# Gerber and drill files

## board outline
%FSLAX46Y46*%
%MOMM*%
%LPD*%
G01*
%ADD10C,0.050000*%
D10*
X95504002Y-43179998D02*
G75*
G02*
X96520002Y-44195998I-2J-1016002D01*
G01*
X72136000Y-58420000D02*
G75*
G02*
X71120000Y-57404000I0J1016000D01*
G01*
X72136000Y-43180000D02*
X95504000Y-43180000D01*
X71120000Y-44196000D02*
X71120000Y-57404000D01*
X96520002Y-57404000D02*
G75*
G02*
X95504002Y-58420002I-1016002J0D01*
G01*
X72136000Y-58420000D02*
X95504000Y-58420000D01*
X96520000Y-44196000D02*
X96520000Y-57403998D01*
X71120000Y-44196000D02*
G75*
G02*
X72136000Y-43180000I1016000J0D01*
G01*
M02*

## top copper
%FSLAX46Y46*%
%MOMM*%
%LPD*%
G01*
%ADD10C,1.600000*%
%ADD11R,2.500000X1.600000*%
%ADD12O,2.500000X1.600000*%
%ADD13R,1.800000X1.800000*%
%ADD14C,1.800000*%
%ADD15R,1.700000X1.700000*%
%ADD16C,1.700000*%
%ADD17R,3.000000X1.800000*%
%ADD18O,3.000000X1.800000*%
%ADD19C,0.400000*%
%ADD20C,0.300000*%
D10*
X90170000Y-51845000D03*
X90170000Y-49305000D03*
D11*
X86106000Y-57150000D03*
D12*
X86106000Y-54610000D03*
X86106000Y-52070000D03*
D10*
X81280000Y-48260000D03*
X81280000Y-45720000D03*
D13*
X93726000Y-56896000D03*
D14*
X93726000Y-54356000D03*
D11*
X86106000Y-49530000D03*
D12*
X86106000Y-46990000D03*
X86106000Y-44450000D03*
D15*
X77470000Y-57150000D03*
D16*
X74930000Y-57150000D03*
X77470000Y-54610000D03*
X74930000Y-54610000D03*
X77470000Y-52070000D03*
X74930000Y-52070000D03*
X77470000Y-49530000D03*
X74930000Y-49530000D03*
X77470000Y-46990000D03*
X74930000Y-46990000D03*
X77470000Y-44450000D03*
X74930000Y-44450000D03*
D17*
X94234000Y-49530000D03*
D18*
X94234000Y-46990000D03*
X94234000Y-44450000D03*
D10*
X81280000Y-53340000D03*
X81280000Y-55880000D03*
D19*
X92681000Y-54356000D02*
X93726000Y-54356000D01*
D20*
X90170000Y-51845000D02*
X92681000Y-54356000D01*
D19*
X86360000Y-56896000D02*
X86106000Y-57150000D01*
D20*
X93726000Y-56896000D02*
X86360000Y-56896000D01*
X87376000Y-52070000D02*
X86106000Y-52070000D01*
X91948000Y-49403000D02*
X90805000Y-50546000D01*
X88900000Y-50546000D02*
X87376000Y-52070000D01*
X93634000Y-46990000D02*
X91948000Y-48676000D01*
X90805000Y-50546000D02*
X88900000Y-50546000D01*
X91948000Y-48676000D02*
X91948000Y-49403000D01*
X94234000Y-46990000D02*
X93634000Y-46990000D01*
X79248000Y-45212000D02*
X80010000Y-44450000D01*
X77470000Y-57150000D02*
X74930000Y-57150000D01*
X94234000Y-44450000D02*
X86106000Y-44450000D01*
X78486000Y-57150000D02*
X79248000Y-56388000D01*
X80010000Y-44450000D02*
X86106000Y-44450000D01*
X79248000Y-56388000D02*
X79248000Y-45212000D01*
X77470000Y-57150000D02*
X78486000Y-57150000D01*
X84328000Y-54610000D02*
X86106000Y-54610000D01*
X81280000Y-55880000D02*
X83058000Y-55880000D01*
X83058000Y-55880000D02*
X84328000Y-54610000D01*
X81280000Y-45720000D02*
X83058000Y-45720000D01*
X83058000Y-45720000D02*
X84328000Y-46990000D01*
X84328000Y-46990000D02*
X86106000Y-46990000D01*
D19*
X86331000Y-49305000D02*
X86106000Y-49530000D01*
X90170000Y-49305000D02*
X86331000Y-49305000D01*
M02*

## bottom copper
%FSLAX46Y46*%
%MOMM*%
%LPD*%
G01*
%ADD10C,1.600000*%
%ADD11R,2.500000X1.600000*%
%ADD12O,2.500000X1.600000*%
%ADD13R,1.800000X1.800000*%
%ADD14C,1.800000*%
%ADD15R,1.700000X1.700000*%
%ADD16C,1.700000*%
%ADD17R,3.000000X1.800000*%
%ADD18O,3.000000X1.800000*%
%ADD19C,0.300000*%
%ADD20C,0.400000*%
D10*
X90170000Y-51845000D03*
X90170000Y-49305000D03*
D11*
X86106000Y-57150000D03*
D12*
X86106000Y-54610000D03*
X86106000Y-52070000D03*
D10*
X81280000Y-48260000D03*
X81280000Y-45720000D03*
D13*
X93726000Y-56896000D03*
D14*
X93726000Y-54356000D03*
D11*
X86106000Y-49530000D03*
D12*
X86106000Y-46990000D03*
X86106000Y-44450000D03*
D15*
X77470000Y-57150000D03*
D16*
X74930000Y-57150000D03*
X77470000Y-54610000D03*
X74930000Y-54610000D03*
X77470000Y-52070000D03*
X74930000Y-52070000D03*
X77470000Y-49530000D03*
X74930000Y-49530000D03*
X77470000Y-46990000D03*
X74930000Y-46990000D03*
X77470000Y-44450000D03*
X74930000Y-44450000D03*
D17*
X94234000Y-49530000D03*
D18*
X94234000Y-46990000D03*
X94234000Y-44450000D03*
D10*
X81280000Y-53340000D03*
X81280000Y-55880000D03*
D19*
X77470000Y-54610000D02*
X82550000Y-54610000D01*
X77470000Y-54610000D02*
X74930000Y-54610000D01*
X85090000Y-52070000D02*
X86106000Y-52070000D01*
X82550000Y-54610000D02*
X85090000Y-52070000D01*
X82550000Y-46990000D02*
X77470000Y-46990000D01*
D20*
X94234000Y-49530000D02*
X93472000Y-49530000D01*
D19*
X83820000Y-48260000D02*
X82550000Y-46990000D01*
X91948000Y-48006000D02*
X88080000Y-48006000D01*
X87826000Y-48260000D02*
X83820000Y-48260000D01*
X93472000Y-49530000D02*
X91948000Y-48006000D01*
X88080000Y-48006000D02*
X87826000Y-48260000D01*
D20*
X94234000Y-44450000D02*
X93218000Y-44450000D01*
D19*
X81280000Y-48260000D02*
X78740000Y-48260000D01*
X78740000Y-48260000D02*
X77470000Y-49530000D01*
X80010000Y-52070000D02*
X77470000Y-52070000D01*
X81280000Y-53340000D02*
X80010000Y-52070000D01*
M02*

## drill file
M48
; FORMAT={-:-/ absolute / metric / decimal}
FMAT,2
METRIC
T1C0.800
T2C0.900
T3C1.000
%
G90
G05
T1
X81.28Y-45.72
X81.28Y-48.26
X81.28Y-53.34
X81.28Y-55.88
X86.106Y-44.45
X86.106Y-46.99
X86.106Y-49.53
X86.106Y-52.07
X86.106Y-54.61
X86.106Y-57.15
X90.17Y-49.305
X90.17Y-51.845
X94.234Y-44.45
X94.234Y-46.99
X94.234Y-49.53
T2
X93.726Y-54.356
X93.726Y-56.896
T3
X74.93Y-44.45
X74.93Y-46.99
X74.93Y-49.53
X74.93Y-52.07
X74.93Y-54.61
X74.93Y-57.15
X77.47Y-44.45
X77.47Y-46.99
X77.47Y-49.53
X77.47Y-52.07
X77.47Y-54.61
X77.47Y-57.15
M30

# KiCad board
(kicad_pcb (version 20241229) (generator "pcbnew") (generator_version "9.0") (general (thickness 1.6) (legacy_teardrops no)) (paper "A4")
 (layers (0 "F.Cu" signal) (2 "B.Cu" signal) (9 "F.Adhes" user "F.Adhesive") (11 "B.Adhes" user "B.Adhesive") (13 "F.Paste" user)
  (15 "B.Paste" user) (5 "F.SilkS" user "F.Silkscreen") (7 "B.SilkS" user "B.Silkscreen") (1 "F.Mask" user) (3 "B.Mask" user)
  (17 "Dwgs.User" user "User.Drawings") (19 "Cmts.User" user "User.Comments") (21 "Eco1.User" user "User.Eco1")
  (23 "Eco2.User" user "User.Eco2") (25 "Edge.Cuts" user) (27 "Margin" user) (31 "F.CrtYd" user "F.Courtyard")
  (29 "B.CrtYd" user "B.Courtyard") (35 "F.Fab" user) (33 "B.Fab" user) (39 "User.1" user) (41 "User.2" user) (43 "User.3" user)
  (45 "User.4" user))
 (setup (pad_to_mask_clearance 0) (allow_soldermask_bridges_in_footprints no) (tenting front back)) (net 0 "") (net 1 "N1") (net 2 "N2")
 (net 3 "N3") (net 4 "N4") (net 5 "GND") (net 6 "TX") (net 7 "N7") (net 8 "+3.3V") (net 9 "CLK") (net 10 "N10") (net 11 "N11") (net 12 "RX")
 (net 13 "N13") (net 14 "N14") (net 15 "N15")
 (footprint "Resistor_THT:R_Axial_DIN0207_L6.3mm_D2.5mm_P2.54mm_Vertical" (layer "F.Cu") (at 90.17 51.845 90)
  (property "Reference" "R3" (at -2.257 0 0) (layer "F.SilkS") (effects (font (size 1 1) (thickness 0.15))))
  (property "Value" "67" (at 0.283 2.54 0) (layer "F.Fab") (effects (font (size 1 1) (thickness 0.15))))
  (pad "1" thru_hole circle (at 0 0 90) (size 1.6 1.6) (drill 0.8) (layers "*.Cu" "*.Mask") (remove_unused_layers no) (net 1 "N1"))
  (pad "2" thru_hole circle (at 2.54 0 90) (size 1.6 1.6) (drill 0.8) (layers "*.Cu" "*.Mask") (remove_unused_layers no) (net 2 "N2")))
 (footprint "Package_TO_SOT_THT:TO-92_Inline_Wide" (layer "F.Cu") (at 86.106 57.15 90)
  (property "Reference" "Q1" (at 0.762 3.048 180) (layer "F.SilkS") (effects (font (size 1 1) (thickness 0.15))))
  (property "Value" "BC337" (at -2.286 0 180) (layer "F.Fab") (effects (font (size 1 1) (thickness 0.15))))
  (pad "1" thru_hole rect (at 0 0 90) (size 1.6 2.5) (drill 0.8) (layers "*.Cu" "*.Mask") (remove_unused_layers no) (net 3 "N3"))
  (pad "2" thru_hole oval (at 2.54 0 90) (size 1.6 2.5) (drill 0.8) (layers "*.Cu" "*.Mask") (remove_unused_layers no) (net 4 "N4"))
  (pad "3" thru_hole oval (at 5.08 0 90) (size 1.6 2.5) (drill 0.8) (layers "*.Cu" "*.Mask") (remove_unused_layers no) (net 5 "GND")))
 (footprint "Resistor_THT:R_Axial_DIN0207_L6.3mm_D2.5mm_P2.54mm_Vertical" (layer "F.Cu") (at 81.28 48.26 90)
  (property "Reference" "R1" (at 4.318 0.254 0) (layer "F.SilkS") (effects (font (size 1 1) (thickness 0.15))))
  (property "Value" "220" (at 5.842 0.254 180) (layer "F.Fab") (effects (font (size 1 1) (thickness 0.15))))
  (pad "1" thru_hole circle (at 0 0 90) (size 1.6 1.6) (drill 0.8) (layers "*.Cu" "*.Mask") (remove_unused_layers no) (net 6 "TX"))
  (pad "2" thru_hole circle (at 2.54 0 90) (size 1.6 1.6) (drill 0.8) (layers "*.Cu" "*.Mask") (remove_unused_layers no) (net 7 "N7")))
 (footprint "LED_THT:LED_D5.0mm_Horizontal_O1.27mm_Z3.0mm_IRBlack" (layer "F.Cu") (at 93.726 56.896 90)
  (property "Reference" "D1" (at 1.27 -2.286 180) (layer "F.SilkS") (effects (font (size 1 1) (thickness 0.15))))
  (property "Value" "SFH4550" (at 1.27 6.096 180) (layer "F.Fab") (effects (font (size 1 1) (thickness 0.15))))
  (pad "1" thru_hole rect (at 0 0 90) (size 1.8 1.8) (drill 0.9) (layers "*.Cu" "*.Mask") (remove_unused_layers no) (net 3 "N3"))
  (pad "2" thru_hole circle (at 2.54 0 90) (size 1.8 1.8) (drill 0.9) (layers "*.Cu" "*.Mask") (remove_unused_layers no) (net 1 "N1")))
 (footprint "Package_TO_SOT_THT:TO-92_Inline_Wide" (layer "F.Cu") (at 86.106 49.53 90)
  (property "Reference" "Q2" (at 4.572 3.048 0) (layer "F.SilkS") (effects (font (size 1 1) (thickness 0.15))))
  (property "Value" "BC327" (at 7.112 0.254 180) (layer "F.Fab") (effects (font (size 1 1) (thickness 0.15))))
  (pad "1" thru_hole rect (at 0 0 90) (size 1.6 2.5) (drill 0.8) (layers "*.Cu" "*.Mask") (remove_unused_layers no) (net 2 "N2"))
  (pad "2" thru_hole oval (at 2.54 0 90) (size 1.6 2.5) (drill 0.8) (layers "*.Cu" "*.Mask") (remove_unused_layers no) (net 7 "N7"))
  (pad "3" thru_hole oval (at 5.08 0 90) (size 1.6 2.5) (drill 0.8) (layers "*.Cu" "*.Mask") (remove_unused_layers no) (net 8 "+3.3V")))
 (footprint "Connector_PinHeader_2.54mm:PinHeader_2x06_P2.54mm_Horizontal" (layer "F.Cu") (at 77.47 57.15 180)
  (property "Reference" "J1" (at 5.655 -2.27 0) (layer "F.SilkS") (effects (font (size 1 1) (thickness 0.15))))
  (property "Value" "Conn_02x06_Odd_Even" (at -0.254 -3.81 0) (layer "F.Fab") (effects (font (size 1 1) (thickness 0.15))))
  (pad "1" thru_hole rect (at 0 0 180) (size 1.7 1.7) (drill 1) (layers "*.Cu" "*.Mask") (remove_unused_layers no) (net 8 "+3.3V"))
  (pad "2" thru_hole circle (at 2.54 0 180) (size 1.7 1.7) (drill 1) (layers "*.Cu" "*.Mask") (remove_unused_layers no) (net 8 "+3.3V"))
  (pad "3" thru_hole circle (at 0 2.54 180) (size 1.7 1.7) (drill 1) (layers "*.Cu" "*.Mask") (remove_unused_layers no) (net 5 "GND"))
  (pad "4" thru_hole circle (at 2.54 2.54 180) (size 1.7 1.7) (drill 1) (layers "*.Cu" "*.Mask") (remove_unused_layers no) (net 5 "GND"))
  (pad "5" thru_hole circle (at 0 5.08 180) (size 1.7 1.7) (drill 1) (layers "*.Cu" "*.Mask") (remove_unused_layers no) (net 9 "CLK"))
  (pad "6" thru_hole circle (at 2.54 5.08 180) (size 1.7 1.7) (drill 1) (layers "*.Cu" "*.Mask") (remove_unused_layers no) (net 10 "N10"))
  (pad "7" thru_hole circle (at 0 7.62 180) (size 1.7 1.7) (drill 1) (layers "*.Cu" "*.Mask") (remove_unused_layers no) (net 6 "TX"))
  (pad "8" thru_hole circle (at 2.54 7.62 180) (size 1.7 1.7) (drill 1) (layers "*.Cu" "*.Mask") (remove_unused_layers no) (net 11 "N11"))
  (pad "9" thru_hole circle (at 0 10.16 180) (size 1.7 1.7) (drill 1) (layers "*.Cu" "*.Mask") (remove_unused_layers no) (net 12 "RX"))
  (pad "10" thru_hole circle (at 2.54 10.16 180) (size 1.7 1.7) (drill 1) (layers "*.Cu" "*.Mask") (remove_unused_layers no) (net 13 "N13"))
  (pad "11" thru_hole circle (at 0 12.7 180) (size 1.7 1.7) (drill 1) (layers "*.Cu" "*.Mask") (remove_unused_layers no) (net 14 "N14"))
  (pad "12" thru_hole circle (at 2.54 12.7 180) (size 1.7 1.7) (drill 1) (layers "*.Cu" "*.Mask") (remove_unused_layers no) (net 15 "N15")))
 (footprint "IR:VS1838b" (layer "F.Cu") (at 94.234 46.99 180)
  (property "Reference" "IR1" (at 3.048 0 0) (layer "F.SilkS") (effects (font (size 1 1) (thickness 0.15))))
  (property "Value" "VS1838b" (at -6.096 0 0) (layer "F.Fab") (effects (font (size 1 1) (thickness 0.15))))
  (pad "1" thru_hole rect (at 0 -2.54 180) (size 3 1.8) (drill 0.8) (layers "*.Cu" "*.Mask") (remove_unused_layers no) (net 12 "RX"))
  (pad "2" thru_hole oval (at 0 0 180) (size 3 1.8) (drill 0.8) (layers "*.Cu" "*.Mask") (remove_unused_layers no) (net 5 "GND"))
  (pad "3" thru_hole oval (at 0 2.54 180) (size 3 1.8) (drill 0.8) (layers "*.Cu" "*.Mask") (remove_unused_layers no) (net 8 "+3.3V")))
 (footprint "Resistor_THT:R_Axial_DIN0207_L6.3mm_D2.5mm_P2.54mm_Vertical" (layer "F.Cu") (at 81.28 53.34 -90)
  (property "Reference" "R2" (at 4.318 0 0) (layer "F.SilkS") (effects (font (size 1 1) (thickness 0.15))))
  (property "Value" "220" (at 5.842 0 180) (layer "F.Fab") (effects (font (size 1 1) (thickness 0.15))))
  (pad "1" thru_hole circle (at 0 0 270) (size 1.6 1.6) (drill 0.8) (layers "*.Cu" "*.Mask") (remove_unused_layers no) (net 9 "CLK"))
  (pad "2" thru_hole circle (at 2.54 0 270) (size 1.6 1.6) (drill 0.8) (layers "*.Cu" "*.Mask") (remove_unused_layers no) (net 4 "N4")))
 (gr_arc (start 95.504002 43.179998) (mid 96.222422 43.477578) (end 96.520002 44.195998) (stroke (width 0.05) (type default))
  (layer "Edge.Cuts"))
 (gr_arc (start 72.136 58.42) (mid 71.41758 58.12242) (end 71.12 57.404) (stroke (width 0.05) (type default)) (layer "Edge.Cuts"))
 (gr_line (start 72.136 43.18) (end 95.504 43.18) (stroke (width 0.05) (type default)) (layer "Edge.Cuts"))
 (gr_line (start 71.12 44.196) (end 71.12 57.404) (stroke (width 0.05) (type default)) (layer "Edge.Cuts"))
 (gr_arc (start 96.520002 57.404) (mid 96.222422 58.12242) (end 95.504002 58.42) (stroke (width 0.05) (type default)) (layer "Edge.Cuts"))
 (gr_line (start 72.136 58.42) (end 95.504 58.42) (stroke (width 0.05) (type default)) (layer "Edge.Cuts"))
 (gr_line (start 96.52 44.196) (end 96.52 57.403998) (stroke (width 0.05) (type default)) (layer "Edge.Cuts"))
 (gr_arc (start 71.12 44.196) (mid 71.41758 43.47758) (end 72.136 43.18) (stroke (width 0.05) (type default)) (layer "Edge.Cuts"))
 (segment (start 92.681 54.356) (end 93.726 54.356) (width 0.4) (layer "F.Cu") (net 1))
 (segment (start 90.17 51.845) (end 92.681 54.356) (width 0.3) (layer "F.Cu") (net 1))
 (segment (start 86.36 56.896) (end 86.106 57.15) (width 0.4) (layer "F.Cu") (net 3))
 (segment (start 93.726 56.896) (end 86.36 56.896) (width 0.3) (layer "F.Cu") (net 3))
 (segment (start 87.376 52.07) (end 86.106 52.07) (width 0.3) (layer "F.Cu") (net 5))
 (segment (start 91.948 49.403) (end 90.805 50.546) (width 0.3) (layer "F.Cu") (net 5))
 (segment (start 88.9 50.546) (end 87.376 52.07) (width 0.3) (layer "F.Cu") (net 5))
 (segment (start 93.634 46.99) (end 91.948 48.676) (width 0.3) (layer "F.Cu") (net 5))
 (segment (start 90.805 50.546) (end 88.9 50.546) (width 0.3) (layer "F.Cu") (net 5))
 (segment (start 91.948 48.676) (end 91.948 49.403) (width 0.3) (layer "F.Cu") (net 5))
 (segment (start 94.234 46.99) (end 93.634 46.99) (width 0.3) (layer "F.Cu") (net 5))
 (segment (start 77.47 54.61) (end 82.55 54.61) (width 0.3) (layer "B.Cu") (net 5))
 (segment (start 77.47 54.61) (end 74.93 54.61) (width 0.3) (layer "B.Cu") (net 5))
 (segment (start 85.09 52.07) (end 86.106 52.07) (width 0.3) (layer "B.Cu") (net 5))
 (segment (start 82.55 54.61) (end 85.09 52.07) (width 0.3) (layer "B.Cu") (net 5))
 (segment (start 82.55 46.99) (end 77.47 46.99) (width 0.3) (layer "B.Cu") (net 12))
 (segment (start 94.234 49.53) (end 93.472 49.53) (width 0.4) (layer "B.Cu") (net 12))
 (segment (start 83.82 48.26) (end 82.55 46.99) (width 0.3) (layer "B.Cu") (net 12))
 (segment (start 91.948 48.006) (end 88.08 48.006) (width 0.3) (layer "B.Cu") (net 12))
 (segment (start 87.826 48.26) (end 83.82 48.26) (width 0.3) (layer "B.Cu") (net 12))
 (segment (start 93.472 49.53) (end 91.948 48.006) (width 0.3) (layer "B.Cu") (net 12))
 (segment (start 88.08 48.006) (end 87.826 48.26) (width 0.3) (layer "B.Cu") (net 12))
 (segment (start 79.248 45.212) (end 80.01 44.45) (width 0.3) (layer "F.Cu") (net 8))
 (segment (start 77.47 57.15) (end 74.93 57.15) (width 0.3) (layer "F.Cu") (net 8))
 (segment (start 94.234 44.45) (end 86.106 44.45) (width 0.3) (layer "F.Cu") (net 8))
 (segment (start 78.486 57.15) (end 79.248 56.388) (width 0.3) (layer "F.Cu") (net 8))
 (segment (start 80.01 44.45) (end 86.106 44.45) (width 0.3) (layer "F.Cu") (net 8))
 (segment (start 79.248 56.388) (end 79.248 45.212) (width 0.3) (layer "F.Cu") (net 8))
 (segment (start 77.47 57.15) (end 78.486 57.15) (width 0.3) (layer "F.Cu") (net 8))
 (segment (start 94.234 44.45) (end 93.218 44.45) (width 0.4) (layer "B.Cu") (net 8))
 (segment (start 84.328 54.61) (end 86.106 54.61) (width 0.3) (layer "F.Cu") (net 4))
 (segment (start 81.28 55.88) (end 83.058 55.88) (width 0.3) (layer "F.Cu") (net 4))
 (segment (start 83.058 55.88) (end 84.328 54.61) (width 0.3) (layer "F.Cu") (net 4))
 (segment (start 81.28 45.72) (end 83.058 45.72) (width 0.3) (layer "F.Cu") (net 7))
 (segment (start 83.058 45.72) (end 84.328 46.99) (width 0.3) (layer "F.Cu") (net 7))
 (segment (start 84.328 46.99) (end 86.106 46.99) (width 0.3) (layer "F.Cu") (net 7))
 (segment (start 86.331 49.305) (end 86.106 49.53) (width 0.4) (layer "F.Cu") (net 2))
 (segment (start 90.17 49.305) (end 86.331 49.305) (width 0.4) (layer "F.Cu") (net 2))
 (segment (start 81.28 48.26) (end 78.74 48.26) (width 0.3) (layer "B.Cu") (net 6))
 (segment (start 78.74 48.26) (end 77.47 49.53) (width 0.3) (layer "B.Cu") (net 6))
 (segment (start 80.01 52.07) (end 77.47 52.07) (width 0.3) (layer "B.Cu") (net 9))
 (segment (start 81.28 53.34) (end 80.01 52.07) (width 0.3) (layer "B.Cu") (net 9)))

